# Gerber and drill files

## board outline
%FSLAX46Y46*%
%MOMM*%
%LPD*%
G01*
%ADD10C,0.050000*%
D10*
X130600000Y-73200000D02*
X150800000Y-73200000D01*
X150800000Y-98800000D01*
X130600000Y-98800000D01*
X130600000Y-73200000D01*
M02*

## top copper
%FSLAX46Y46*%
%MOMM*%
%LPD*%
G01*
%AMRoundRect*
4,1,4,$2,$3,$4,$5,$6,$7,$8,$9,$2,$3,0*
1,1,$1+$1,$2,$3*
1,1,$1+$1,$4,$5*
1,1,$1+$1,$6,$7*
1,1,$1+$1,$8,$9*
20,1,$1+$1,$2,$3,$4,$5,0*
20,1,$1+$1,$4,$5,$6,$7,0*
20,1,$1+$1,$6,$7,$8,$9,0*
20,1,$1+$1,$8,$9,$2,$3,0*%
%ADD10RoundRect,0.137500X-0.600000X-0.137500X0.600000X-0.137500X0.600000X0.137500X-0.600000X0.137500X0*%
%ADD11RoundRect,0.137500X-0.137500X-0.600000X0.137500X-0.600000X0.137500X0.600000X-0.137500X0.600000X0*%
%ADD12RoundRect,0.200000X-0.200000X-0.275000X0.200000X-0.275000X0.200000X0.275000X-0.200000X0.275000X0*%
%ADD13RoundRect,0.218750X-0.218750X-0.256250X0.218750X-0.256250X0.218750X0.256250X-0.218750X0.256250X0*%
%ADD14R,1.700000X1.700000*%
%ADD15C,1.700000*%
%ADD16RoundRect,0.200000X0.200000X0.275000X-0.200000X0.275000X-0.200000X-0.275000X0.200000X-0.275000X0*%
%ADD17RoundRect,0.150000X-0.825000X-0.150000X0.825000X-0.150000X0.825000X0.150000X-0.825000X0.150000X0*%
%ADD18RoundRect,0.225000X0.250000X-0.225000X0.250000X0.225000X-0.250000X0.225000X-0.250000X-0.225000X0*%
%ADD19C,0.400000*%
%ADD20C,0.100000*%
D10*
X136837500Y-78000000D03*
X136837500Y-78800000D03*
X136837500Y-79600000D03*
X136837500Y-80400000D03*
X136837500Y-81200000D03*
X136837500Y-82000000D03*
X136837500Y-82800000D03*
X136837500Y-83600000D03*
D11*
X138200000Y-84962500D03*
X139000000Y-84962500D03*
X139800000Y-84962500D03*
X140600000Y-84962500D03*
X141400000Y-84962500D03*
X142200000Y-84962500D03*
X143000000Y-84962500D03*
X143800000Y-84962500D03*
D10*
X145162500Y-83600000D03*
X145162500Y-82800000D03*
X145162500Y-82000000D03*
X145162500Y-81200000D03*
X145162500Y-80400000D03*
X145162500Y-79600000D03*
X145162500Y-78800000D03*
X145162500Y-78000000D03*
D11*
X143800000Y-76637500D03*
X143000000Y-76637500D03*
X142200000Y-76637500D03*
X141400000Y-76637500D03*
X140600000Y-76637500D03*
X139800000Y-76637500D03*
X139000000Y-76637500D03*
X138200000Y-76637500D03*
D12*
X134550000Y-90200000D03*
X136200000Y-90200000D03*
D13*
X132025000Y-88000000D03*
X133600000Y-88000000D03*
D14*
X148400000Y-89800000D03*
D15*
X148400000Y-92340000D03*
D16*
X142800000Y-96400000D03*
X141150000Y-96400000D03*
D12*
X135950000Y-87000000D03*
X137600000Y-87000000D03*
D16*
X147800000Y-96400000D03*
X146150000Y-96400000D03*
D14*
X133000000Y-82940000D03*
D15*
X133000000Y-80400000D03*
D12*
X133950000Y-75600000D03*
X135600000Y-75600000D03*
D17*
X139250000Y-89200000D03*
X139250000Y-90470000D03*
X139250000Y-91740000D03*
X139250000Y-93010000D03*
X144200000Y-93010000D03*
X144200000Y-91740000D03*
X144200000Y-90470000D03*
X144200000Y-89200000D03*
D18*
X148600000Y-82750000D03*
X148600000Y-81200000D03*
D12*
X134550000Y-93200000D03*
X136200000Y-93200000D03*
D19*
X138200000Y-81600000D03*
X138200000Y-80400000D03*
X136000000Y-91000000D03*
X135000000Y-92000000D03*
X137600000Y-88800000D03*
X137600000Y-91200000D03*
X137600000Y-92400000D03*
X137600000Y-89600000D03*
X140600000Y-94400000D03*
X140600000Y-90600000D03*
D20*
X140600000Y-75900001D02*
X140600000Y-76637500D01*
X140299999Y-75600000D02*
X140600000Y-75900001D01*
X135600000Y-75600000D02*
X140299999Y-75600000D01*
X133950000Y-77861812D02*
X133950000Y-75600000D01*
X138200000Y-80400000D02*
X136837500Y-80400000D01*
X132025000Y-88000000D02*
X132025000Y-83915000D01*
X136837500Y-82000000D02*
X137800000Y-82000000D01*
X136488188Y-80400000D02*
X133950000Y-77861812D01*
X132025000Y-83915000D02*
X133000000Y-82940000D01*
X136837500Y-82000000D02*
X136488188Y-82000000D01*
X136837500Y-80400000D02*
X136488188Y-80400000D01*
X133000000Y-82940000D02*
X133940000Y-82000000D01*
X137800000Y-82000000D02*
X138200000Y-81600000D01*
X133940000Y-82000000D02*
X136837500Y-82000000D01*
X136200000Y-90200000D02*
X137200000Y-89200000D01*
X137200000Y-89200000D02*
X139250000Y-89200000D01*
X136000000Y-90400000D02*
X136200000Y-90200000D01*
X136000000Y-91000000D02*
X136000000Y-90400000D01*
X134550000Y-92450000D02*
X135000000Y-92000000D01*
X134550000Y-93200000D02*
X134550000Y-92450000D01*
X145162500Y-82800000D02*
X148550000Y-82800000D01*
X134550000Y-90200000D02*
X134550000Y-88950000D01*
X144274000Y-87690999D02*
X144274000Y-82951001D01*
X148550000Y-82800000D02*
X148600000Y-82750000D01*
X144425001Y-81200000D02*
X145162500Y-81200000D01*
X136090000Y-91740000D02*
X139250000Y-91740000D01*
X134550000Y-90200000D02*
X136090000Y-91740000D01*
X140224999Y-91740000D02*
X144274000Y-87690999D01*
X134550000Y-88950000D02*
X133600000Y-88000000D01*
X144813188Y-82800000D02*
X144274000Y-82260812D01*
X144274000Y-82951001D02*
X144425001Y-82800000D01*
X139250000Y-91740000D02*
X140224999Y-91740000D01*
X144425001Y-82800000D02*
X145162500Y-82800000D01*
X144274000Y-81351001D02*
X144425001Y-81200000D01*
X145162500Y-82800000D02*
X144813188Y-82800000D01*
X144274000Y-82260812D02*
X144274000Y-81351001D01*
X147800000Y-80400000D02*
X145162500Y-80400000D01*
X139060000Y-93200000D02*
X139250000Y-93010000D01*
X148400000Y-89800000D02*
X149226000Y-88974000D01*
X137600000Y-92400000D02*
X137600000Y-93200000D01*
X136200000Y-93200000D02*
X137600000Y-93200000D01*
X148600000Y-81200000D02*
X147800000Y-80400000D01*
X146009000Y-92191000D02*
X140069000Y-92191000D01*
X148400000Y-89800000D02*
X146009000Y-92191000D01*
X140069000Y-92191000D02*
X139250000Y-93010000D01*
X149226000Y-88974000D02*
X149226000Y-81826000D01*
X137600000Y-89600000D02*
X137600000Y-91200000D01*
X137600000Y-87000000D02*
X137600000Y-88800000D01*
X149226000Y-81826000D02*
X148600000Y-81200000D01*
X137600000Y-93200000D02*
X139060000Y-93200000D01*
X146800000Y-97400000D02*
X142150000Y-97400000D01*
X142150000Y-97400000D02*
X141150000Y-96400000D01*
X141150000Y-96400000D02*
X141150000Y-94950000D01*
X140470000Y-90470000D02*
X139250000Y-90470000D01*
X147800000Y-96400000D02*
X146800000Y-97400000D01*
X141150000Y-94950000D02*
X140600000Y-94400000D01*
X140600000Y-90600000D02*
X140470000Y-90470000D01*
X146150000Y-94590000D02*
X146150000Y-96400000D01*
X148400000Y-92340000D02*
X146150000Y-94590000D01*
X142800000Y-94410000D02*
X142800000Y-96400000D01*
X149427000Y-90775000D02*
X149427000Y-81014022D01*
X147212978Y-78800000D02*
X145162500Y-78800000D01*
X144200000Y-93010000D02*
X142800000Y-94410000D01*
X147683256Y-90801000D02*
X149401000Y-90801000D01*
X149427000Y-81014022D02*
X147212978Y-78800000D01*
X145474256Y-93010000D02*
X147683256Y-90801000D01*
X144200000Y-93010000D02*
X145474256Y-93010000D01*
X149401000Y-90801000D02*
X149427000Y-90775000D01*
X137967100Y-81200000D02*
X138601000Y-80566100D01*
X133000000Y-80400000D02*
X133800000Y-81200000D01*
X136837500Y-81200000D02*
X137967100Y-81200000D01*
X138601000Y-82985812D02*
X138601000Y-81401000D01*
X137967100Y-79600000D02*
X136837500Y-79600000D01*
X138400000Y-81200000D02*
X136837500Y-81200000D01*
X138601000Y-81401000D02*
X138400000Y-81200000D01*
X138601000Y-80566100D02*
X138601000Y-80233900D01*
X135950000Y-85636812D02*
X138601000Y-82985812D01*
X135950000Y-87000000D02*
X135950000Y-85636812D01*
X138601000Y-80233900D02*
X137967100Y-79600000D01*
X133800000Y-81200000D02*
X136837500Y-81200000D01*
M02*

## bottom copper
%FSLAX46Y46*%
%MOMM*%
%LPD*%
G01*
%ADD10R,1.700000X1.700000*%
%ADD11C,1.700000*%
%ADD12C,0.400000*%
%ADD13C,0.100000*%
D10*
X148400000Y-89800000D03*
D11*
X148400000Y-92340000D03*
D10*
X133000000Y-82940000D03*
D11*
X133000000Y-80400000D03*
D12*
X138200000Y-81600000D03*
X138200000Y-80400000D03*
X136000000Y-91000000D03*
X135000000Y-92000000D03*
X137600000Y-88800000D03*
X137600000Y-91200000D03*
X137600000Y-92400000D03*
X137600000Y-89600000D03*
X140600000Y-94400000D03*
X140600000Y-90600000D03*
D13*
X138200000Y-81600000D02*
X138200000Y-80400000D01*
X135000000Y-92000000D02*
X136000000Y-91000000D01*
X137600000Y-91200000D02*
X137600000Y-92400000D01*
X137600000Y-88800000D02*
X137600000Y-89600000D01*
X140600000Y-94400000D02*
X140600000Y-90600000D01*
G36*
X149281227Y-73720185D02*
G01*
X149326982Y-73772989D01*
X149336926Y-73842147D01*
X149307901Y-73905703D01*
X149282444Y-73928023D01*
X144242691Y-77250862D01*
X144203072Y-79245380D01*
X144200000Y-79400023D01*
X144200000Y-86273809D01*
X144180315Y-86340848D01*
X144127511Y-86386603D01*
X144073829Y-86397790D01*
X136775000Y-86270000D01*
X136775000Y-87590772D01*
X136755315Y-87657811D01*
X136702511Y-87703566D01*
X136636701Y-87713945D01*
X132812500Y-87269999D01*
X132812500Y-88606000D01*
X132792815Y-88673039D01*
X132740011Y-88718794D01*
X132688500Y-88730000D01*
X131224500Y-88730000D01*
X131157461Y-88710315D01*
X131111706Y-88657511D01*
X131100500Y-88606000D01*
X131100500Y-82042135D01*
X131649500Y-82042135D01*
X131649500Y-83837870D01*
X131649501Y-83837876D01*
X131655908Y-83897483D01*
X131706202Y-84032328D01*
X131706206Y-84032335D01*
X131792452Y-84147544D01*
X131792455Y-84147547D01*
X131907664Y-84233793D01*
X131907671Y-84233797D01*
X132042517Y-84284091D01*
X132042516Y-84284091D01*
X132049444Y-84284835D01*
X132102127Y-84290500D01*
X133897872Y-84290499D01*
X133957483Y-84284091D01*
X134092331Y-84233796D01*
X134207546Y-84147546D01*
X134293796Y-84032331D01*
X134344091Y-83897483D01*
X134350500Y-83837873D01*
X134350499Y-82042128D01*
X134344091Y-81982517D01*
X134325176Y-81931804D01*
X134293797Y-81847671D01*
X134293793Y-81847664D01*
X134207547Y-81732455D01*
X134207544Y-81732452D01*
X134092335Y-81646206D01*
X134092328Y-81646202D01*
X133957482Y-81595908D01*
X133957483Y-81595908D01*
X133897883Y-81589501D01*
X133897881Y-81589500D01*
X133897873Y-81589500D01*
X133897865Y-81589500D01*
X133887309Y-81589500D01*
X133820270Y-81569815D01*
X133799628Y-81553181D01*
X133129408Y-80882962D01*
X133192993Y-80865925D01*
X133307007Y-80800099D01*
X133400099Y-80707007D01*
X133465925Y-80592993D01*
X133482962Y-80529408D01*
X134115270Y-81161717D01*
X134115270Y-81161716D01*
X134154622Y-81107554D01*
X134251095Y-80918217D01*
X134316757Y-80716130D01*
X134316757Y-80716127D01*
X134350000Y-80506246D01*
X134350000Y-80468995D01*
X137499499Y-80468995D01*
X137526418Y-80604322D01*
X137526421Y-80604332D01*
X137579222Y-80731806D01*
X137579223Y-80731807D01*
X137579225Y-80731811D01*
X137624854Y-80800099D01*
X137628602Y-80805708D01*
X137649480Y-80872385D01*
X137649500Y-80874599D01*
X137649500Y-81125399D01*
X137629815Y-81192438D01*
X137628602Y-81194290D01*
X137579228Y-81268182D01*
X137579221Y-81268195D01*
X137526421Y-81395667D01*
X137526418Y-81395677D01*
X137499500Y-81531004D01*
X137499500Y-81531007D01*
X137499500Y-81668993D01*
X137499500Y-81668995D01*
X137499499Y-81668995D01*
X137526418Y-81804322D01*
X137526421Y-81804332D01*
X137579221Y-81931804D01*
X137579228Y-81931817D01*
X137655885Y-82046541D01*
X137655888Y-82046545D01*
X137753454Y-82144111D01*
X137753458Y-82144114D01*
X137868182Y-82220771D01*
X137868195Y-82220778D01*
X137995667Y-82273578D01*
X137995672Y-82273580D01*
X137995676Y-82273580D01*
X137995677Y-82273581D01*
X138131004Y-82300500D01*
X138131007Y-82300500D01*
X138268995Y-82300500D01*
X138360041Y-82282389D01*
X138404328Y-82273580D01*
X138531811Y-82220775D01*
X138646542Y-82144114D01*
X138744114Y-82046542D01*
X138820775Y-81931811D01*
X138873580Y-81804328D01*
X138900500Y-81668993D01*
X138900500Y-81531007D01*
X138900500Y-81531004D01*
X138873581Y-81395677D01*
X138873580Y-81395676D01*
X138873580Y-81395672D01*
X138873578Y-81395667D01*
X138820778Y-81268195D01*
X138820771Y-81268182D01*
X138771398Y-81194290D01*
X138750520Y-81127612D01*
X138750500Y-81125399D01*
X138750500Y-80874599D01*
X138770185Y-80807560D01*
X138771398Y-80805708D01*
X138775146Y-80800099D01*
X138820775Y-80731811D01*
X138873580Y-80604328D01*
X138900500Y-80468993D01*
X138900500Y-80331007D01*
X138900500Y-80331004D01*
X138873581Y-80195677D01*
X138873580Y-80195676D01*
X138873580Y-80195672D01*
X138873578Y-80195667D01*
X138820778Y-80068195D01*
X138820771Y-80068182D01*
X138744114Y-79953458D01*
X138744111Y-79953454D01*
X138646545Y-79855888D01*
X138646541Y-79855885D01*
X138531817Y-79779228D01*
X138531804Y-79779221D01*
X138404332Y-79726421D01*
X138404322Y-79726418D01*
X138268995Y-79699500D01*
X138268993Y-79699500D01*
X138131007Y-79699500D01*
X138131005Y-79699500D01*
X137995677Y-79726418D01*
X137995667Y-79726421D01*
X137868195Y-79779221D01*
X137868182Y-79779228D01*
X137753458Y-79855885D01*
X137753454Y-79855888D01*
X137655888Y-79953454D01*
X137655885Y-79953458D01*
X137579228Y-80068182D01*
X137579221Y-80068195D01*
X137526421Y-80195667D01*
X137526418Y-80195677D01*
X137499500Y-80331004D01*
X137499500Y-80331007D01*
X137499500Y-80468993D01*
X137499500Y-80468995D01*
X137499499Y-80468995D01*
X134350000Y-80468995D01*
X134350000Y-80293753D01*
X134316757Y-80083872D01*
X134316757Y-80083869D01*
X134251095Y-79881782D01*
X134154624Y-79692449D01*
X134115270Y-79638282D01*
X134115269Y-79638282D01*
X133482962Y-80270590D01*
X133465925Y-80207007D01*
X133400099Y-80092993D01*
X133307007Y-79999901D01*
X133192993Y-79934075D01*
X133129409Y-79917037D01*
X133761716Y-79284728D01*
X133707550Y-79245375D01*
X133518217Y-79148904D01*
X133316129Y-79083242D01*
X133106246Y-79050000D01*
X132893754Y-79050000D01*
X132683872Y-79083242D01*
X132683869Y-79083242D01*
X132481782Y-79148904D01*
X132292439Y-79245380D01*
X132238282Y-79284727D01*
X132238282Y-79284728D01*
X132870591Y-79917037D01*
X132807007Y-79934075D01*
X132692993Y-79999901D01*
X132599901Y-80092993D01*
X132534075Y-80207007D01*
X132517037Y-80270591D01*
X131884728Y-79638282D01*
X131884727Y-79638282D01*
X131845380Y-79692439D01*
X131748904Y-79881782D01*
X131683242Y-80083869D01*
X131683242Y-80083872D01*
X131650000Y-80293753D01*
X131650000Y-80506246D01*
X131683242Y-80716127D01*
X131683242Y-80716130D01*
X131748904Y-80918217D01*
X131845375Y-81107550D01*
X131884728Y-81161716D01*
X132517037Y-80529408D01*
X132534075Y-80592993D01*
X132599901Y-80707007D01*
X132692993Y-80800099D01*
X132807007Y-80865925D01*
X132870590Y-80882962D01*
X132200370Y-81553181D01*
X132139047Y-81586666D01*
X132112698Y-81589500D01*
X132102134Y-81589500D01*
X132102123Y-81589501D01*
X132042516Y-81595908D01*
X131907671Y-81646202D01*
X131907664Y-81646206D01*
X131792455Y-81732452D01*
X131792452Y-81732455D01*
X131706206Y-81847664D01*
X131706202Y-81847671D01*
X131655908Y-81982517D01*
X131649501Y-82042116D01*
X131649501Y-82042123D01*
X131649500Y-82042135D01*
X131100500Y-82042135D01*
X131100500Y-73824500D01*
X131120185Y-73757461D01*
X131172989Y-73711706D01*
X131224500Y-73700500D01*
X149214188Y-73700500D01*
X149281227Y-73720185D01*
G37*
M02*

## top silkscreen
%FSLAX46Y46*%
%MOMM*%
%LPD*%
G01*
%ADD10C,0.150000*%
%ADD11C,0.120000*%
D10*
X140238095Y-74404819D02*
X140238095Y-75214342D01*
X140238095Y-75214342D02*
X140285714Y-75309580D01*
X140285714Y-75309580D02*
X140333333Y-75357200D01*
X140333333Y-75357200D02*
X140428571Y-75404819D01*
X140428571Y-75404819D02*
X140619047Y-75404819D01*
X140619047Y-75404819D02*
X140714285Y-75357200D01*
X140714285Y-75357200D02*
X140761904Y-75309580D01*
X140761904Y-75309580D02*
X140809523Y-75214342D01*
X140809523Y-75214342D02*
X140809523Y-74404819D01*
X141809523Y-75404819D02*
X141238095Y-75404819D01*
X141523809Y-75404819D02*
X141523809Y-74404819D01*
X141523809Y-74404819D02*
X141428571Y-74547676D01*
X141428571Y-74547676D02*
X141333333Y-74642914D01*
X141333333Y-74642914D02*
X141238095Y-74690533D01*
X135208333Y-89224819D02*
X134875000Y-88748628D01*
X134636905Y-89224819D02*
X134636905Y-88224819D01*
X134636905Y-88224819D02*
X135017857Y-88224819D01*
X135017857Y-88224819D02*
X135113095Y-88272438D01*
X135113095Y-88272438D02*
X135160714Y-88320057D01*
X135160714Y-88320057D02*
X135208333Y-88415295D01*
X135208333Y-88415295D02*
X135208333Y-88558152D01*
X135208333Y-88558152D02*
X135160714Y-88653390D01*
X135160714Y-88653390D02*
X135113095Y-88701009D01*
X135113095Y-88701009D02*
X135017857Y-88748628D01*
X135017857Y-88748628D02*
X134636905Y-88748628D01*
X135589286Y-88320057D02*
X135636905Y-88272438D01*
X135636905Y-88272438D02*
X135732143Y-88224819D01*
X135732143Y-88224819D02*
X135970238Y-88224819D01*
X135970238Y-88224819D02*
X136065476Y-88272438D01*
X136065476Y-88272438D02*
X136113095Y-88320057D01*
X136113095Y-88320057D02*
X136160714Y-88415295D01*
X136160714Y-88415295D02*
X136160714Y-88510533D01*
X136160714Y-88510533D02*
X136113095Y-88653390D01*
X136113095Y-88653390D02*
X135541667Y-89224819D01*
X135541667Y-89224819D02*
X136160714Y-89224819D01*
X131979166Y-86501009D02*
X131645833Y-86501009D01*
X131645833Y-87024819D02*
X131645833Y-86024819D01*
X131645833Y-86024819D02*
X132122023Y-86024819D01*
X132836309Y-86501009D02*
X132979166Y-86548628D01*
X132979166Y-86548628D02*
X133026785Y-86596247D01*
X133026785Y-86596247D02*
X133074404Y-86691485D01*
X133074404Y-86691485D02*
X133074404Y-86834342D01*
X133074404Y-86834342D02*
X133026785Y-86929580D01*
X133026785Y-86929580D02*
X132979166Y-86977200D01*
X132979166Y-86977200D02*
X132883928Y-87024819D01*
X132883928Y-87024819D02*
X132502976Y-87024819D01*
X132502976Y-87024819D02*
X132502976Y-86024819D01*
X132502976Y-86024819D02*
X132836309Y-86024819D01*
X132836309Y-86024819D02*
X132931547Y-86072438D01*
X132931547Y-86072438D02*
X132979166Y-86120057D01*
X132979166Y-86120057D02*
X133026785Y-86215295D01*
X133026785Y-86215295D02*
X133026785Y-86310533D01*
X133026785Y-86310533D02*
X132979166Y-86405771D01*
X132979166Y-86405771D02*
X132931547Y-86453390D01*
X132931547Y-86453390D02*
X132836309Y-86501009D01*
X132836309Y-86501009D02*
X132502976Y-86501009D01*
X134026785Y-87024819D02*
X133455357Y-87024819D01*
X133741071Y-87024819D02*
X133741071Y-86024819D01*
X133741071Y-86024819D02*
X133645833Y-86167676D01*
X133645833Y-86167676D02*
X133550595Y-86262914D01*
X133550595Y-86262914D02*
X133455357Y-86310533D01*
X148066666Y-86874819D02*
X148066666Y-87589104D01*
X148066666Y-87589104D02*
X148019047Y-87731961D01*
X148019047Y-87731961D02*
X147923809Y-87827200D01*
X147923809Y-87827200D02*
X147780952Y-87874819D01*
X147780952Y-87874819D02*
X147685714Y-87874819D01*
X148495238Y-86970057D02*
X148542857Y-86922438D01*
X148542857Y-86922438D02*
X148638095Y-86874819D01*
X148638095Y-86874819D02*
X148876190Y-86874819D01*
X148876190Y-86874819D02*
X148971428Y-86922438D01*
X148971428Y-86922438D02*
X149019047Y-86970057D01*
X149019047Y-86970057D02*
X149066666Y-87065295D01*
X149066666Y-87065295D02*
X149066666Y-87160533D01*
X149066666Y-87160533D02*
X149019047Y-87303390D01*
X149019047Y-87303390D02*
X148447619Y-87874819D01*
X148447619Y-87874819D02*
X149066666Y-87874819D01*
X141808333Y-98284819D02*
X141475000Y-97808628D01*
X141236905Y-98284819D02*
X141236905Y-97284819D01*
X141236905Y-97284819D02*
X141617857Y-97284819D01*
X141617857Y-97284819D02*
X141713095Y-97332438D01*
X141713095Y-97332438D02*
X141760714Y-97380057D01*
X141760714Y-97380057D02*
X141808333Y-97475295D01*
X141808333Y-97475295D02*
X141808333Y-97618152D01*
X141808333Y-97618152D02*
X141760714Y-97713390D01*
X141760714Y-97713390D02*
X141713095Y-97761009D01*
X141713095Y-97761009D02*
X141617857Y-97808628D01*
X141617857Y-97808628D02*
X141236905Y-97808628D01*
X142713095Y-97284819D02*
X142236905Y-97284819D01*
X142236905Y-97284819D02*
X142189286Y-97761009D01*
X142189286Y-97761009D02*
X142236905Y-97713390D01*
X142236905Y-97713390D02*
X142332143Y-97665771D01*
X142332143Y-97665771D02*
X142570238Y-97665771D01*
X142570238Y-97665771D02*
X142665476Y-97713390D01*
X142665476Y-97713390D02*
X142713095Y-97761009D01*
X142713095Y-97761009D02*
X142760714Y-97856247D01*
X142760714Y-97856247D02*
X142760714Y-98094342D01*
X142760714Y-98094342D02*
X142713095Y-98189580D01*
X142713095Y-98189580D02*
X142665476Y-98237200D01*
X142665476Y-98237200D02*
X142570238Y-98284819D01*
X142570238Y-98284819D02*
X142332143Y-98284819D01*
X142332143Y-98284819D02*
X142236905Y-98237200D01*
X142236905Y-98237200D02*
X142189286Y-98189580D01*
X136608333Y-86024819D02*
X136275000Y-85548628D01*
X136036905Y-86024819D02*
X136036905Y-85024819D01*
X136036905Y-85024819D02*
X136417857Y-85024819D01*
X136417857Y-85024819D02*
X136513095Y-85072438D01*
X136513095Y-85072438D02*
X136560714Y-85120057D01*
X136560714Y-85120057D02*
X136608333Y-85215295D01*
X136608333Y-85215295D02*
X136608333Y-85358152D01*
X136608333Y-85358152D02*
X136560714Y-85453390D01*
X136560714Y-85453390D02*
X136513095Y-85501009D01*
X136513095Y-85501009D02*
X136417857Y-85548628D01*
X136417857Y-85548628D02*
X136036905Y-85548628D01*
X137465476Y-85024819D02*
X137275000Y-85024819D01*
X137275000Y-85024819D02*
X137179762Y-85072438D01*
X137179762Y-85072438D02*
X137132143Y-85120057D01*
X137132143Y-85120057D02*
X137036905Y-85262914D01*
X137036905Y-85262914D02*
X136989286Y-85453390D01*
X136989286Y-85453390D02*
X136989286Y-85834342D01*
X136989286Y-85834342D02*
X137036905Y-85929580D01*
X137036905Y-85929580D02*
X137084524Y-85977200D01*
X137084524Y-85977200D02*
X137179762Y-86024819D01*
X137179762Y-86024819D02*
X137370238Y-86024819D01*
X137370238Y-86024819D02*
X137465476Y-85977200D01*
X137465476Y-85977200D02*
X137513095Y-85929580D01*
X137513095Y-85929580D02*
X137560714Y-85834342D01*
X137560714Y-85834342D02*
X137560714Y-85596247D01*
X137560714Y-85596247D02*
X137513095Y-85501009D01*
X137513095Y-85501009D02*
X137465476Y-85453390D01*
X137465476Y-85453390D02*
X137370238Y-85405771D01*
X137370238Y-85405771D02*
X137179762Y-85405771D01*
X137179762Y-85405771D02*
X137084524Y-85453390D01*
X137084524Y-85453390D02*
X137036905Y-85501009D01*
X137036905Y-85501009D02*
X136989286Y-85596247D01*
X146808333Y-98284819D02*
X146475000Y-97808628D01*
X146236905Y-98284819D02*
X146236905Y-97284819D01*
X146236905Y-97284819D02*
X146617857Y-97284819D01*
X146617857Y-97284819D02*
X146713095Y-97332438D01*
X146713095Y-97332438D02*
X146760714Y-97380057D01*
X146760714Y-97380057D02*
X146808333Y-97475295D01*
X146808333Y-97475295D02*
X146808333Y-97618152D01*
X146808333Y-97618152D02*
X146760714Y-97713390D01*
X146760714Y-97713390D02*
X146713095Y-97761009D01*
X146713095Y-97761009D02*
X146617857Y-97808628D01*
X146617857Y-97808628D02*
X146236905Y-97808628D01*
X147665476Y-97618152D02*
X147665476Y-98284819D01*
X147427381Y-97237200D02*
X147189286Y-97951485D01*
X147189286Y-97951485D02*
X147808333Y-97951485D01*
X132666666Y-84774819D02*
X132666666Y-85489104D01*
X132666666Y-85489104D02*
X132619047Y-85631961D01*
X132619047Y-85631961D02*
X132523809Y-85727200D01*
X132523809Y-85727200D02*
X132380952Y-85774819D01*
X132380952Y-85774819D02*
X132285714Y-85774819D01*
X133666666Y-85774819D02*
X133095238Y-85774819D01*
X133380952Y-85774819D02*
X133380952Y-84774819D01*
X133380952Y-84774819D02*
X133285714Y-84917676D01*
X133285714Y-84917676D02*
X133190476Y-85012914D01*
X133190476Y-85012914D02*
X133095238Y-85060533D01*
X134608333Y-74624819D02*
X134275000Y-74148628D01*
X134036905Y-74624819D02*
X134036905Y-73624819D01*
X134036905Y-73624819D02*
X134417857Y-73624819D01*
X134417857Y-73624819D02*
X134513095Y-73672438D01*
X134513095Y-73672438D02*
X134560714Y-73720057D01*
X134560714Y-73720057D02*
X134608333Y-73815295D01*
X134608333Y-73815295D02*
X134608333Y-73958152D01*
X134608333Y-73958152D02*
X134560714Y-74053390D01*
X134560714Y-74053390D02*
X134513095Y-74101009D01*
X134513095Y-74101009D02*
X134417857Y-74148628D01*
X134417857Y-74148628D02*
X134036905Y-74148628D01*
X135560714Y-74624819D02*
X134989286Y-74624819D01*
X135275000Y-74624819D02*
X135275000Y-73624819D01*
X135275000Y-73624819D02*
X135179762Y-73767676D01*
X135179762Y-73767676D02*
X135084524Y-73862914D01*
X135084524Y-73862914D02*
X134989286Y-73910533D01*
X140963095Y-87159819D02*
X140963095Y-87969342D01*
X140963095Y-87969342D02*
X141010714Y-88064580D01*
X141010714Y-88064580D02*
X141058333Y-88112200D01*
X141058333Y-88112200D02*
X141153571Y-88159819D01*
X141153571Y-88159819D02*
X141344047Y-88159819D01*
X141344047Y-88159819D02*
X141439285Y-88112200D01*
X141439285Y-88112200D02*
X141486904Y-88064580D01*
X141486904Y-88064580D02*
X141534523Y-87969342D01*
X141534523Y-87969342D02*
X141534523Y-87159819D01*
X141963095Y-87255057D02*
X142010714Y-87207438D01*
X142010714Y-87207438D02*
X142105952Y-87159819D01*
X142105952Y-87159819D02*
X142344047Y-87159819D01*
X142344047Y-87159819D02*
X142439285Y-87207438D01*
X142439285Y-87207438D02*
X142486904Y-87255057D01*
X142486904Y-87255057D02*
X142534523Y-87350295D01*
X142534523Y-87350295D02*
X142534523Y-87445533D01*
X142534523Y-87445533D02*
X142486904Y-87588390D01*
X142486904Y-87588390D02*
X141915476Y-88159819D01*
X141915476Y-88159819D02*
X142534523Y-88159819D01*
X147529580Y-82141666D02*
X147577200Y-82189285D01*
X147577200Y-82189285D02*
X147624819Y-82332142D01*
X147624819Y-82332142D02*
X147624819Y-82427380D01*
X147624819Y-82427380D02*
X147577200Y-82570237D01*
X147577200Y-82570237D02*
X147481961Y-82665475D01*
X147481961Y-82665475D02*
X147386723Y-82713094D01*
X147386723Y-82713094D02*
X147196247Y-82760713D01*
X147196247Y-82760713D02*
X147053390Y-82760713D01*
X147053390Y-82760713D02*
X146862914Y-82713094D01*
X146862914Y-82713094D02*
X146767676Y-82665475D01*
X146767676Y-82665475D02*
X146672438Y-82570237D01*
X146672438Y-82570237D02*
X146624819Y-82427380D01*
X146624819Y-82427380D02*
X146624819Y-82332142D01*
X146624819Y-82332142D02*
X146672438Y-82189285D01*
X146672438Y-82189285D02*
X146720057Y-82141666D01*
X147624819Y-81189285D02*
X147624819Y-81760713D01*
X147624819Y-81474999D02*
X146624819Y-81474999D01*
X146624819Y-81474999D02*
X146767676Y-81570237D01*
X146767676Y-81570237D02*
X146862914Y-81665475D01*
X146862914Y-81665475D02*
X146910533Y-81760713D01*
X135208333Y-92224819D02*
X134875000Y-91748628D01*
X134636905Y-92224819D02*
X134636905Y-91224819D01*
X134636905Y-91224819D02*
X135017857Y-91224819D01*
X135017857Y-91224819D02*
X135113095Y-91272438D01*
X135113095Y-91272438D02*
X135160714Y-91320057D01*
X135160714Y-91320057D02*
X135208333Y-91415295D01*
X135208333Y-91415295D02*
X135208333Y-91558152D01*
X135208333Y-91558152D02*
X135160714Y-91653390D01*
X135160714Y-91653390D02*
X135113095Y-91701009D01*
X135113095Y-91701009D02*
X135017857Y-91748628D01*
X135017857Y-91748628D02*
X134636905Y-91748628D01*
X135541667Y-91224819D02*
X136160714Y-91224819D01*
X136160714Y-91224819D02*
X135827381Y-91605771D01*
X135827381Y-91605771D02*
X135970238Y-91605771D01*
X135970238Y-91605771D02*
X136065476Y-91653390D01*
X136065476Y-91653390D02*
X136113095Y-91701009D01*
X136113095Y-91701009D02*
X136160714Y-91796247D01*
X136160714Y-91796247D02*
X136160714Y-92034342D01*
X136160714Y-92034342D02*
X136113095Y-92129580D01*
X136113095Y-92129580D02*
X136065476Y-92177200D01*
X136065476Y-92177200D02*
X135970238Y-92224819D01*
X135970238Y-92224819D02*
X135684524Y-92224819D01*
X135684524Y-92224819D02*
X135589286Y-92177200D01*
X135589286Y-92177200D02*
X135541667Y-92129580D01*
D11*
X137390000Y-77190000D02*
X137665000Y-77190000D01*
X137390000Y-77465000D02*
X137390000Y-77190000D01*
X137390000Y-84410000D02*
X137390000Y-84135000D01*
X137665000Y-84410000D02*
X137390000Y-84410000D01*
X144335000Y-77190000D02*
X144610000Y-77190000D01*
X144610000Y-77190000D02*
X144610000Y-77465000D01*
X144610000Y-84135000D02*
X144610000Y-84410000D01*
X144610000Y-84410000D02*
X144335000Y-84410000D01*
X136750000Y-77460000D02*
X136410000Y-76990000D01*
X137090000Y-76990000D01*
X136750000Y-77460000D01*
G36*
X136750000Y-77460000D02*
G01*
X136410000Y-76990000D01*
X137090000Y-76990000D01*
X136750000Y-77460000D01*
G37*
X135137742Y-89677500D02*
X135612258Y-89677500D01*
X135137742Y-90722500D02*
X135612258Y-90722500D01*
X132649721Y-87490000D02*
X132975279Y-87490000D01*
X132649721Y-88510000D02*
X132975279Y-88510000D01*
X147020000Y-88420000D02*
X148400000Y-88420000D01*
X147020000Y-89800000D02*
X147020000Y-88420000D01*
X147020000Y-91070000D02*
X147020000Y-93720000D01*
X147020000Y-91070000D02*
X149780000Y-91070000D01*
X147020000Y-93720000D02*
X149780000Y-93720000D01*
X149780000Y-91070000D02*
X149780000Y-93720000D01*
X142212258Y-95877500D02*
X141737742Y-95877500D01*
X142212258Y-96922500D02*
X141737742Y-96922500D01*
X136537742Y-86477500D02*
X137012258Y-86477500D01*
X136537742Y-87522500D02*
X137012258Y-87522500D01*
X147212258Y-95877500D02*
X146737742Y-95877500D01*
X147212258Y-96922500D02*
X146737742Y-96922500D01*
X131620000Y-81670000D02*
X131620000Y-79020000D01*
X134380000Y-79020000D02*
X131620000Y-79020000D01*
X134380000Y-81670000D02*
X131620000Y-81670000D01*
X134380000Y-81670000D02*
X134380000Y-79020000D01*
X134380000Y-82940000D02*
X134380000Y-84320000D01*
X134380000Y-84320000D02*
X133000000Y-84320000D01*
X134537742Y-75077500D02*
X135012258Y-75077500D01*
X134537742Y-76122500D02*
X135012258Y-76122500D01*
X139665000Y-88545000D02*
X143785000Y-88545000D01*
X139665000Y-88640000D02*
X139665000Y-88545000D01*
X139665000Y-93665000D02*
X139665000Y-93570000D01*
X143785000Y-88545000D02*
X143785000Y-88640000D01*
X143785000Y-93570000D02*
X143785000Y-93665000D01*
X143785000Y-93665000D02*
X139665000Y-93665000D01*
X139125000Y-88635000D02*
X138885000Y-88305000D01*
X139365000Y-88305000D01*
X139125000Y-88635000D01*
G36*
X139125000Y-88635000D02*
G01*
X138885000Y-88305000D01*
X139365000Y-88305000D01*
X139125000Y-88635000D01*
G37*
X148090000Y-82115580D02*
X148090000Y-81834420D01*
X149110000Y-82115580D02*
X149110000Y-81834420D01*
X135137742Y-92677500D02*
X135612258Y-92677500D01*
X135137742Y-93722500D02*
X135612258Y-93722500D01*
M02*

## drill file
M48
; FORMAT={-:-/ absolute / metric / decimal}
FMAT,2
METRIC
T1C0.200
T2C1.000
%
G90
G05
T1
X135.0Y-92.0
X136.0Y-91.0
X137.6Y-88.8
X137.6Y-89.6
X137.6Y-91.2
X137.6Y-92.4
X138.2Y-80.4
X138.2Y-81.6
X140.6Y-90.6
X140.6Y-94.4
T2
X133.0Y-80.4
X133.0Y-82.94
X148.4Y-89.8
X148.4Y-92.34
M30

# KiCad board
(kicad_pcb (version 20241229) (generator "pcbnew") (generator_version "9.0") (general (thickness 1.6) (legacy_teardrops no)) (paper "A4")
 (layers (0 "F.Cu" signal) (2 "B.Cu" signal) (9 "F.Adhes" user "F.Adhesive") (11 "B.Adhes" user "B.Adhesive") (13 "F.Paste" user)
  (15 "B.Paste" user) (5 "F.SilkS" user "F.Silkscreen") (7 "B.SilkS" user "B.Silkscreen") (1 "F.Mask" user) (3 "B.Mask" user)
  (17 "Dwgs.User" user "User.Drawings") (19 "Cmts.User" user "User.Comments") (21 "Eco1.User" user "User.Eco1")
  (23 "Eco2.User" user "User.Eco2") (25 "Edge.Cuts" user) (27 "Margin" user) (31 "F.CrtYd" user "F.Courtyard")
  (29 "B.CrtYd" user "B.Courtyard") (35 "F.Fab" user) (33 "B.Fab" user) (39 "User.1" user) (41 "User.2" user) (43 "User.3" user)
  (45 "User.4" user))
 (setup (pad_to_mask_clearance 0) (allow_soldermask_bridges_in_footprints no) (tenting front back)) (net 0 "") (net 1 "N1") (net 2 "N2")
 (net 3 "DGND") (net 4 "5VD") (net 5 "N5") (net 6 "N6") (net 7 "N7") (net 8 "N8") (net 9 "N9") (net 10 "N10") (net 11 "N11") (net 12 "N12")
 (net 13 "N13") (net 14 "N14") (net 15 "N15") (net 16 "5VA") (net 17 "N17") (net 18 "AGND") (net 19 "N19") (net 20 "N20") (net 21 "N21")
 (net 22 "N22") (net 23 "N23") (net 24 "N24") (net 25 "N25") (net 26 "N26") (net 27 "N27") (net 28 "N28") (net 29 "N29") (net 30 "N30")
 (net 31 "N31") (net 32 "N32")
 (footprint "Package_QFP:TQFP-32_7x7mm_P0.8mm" (layer "F.Cu") (at 141 80.8)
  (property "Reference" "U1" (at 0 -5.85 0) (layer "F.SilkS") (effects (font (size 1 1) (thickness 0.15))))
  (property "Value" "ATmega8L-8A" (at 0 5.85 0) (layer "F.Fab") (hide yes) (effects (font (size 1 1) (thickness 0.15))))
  (fp_line (start -3.61 -3.61) (end -3.335 -3.61) (stroke (width 0.12) (type solid)) (layer "F.SilkS"))
  (fp_line (start -3.61 -3.335) (end -3.61 -3.61) (stroke (width 0.12) (type solid)) (layer "F.SilkS"))
  (fp_line (start -3.61 3.61) (end -3.61 3.335) (stroke (width 0.12) (type solid)) (layer "F.SilkS"))
  (fp_line (start -3.335 3.61) (end -3.61 3.61) (stroke (width 0.12) (type solid)) (layer "F.SilkS"))
  (fp_line (start 3.335 -3.61) (end 3.61 -3.61) (stroke (width 0.12) (type solid)) (layer "F.SilkS"))
  (fp_line (start 3.61 -3.61) (end 3.61 -3.335) (stroke (width 0.12) (type solid)) (layer "F.SilkS"))
  (fp_line (start 3.61 3.335) (end 3.61 3.61) (stroke (width 0.12) (type solid)) (layer "F.SilkS"))
  (fp_line (start 3.61 3.61) (end 3.335 3.61) (stroke (width 0.12) (type solid)) (layer "F.SilkS"))
  (fp_poly (pts (xy -4.25 -3.34) (xy -4.59 -3.81) (xy -3.91 -3.81)) (stroke (width 0.12) (type solid)) (fill yes) (layer "F.SilkS"))
  (pad "1" smd roundrect (at -4.1625 -2.8) (size 1.475 0.55) (layers "F.Cu" "F.Mask" "F.Paste") (roundrect_rratio 0.25) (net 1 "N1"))
  (pad "2" smd roundrect (at -4.1625 -2) (size 1.475 0.55) (layers "F.Cu" "F.Mask" "F.Paste") (roundrect_rratio 0.25) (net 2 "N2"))
  (pad "3" smd roundrect (at -4.1625 -1.2) (size 1.475 0.55) (layers "F.Cu" "F.Mask" "F.Paste") (roundrect_rratio 0.25) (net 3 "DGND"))
  (pad "4" smd roundrect (at -4.1625 -0.4) (size 1.475 0.55) (layers "F.Cu" "F.Mask" "F.Paste") (roundrect_rratio 0.25) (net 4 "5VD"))
  (pad "5" smd roundrect (at -4.1625 0.4) (size 1.475 0.55) (layers "F.Cu" "F.Mask" "F.Paste") (roundrect_rratio 0.25) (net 3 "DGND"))
  (pad "6" smd roundrect (at -4.1625 1.2) (size 1.475 0.55) (layers "F.Cu" "F.Mask" "F.Paste") (roundrect_rratio 0.25) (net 4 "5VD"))
  (pad "7" smd roundrect (at -4.1625 2) (size 1.475 0.55) (layers "F.Cu" "F.Mask" "F.Paste") (roundrect_rratio 0.25) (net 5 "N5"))
  (pad "8" smd roundrect (at -4.1625 2.8) (size 1.475 0.55) (layers "F.Cu" "F.Mask" "F.Paste") (roundrect_rratio 0.25) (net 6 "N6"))
  (pad "9" smd roundrect (at -2.8 4.1625) (size 0.55 1.475) (layers "F.Cu" "F.Mask" "F.Paste") (roundrect_rratio 0.25) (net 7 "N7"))
  (pad "10" smd roundrect (at -2 4.1625) (size 0.55 1.475) (layers "F.Cu" "F.Mask" "F.Paste") (roundrect_rratio 0.25) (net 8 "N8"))
  (pad "11" smd roundrect (at -1.2 4.1625) (size 0.55 1.475) (layers "F.Cu" "F.Mask" "F.Paste") (roundrect_rratio 0.25) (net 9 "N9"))
  (pad "12" smd roundrect (at -0.4 4.1625) (size 0.55 1.475) (layers "F.Cu" "F.Mask" "F.Paste") (roundrect_rratio 0.25) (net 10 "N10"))
  (pad "13" smd roundrect (at 0.4 4.1625) (size 0.55 1.475) (layers "F.Cu" "F.Mask" "F.Paste") (roundrect_rratio 0.25) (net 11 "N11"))
  (pad "14" smd roundrect (at 1.2 4.1625) (size 0.55 1.475) (layers "F.Cu" "F.Mask" "F.Paste") (roundrect_rratio 0.25) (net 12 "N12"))
  (pad "15" smd roundrect (at 2 4.1625) (size 0.55 1.475) (layers "F.Cu" "F.Mask" "F.Paste") (roundrect_rratio 0.25) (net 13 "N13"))
  (pad "16" smd roundrect (at 2.8 4.1625) (size 0.55 1.475) (layers "F.Cu" "F.Mask" "F.Paste") (roundrect_rratio 0.25) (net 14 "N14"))
  (pad "17" smd roundrect (at 4.1625 2.8) (size 1.475 0.55) (layers "F.Cu" "F.Mask" "F.Paste") (roundrect_rratio 0.25) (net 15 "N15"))
  (pad "18" smd roundrect (at 4.1625 2) (size 1.475 0.55) (layers "F.Cu" "F.Mask" "F.Paste") (roundrect_rratio 0.25) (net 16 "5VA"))
  (pad "19" smd roundrect (at 4.1625 1.2) (size 1.475 0.55) (layers "F.Cu" "F.Mask" "F.Paste") (roundrect_rratio 0.25) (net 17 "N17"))
  (pad "20" smd roundrect (at 4.1625 0.4) (size 1.475 0.55) (layers "F.Cu" "F.Mask" "F.Paste") (roundrect_rratio 0.25) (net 16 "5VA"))
  (pad "21" smd roundrect (at 4.1625 -0.4) (size 1.475 0.55) (layers "F.Cu" "F.Mask" "F.Paste") (roundrect_rratio 0.25) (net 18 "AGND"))
  (pad "22" smd roundrect (at 4.1625 -1.2) (size 1.475 0.55) (layers "F.Cu" "F.Mask" "F.Paste") (roundrect_rratio 0.25) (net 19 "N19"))
  (pad "23" smd roundrect (at 4.1625 -2) (size 1.475 0.55) (layers "F.Cu" "F.Mask" "F.Paste") (roundrect_rratio 0.25) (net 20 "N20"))
  (pad "24" smd roundrect (at 4.1625 -2.8) (size 1.475 0.55) (layers "F.Cu" "F.Mask" "F.Paste") (roundrect_rratio 0.25) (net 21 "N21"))
  (pad "25" smd roundrect (at 2.8 -4.1625) (size 0.55 1.475) (layers "F.Cu" "F.Mask" "F.Paste") (roundrect_rratio 0.25) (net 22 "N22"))
  (pad "26" smd roundrect (at 2 -4.1625) (size 0.55 1.475) (layers "F.Cu" "F.Mask" "F.Paste") (roundrect_rratio 0.25) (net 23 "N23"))
  (pad "27" smd roundrect (at 1.2 -4.1625) (size 0.55 1.475) (layers "F.Cu" "F.Mask" "F.Paste") (roundrect_rratio 0.25) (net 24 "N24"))
  (pad "28" smd roundrect (at 0.4 -4.1625) (size 0.55 1.475) (layers "F.Cu" "F.Mask" "F.Paste") (roundrect_rratio 0.25) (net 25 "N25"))
  (pad "29" smd roundrect (at -0.4 -4.1625) (size 0.55 1.475) (layers "F.Cu" "F.Mask" "F.Paste") (roundrect_rratio 0.25) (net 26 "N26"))
  (pad "30" smd roundrect (at -1.2 -4.1625) (size 0.55 1.475) (layers "F.Cu" "F.Mask" "F.Paste") (roundrect_rratio 0.25) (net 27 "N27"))
  (pad "31" smd roundrect (at -2 -4.1625) (size 0.55 1.475) (layers "F.Cu" "F.Mask" "F.Paste") (roundrect_rratio 0.25) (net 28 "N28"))
  (pad "32" smd roundrect (at -2.8 -4.1625) (size 0.55 1.475) (layers "F.Cu" "F.Mask" "F.Paste") (roundrect_rratio 0.25) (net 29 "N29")))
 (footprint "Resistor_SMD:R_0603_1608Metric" (layer "F.Cu") (at 135.375 90.2)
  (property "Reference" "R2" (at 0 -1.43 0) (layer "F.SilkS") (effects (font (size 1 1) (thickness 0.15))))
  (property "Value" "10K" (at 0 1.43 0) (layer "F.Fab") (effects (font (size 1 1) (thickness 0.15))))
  (fp_line (start -0.237258 -0.5225) (end 0.237258 -0.5225) (stroke (width 0.12) (type solid)) (layer "F.SilkS"))
  (fp_line (start -0.237258 0.5225) (end 0.237258 0.5225) (stroke (width 0.12) (type solid)) (layer "F.SilkS"))
  (pad "1" smd roundrect (at -0.825 0) (size 0.8 0.95) (layers "F.Cu" "F.Mask" "F.Paste") (roundrect_rratio 0.25) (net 16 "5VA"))
  (pad "2" smd roundrect (at 0.825 0) (size 0.8 0.95) (layers "F.Cu" "F.Mask" "F.Paste") (roundrect_rratio 0.25) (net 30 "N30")))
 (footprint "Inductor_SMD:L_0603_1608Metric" (layer "F.Cu") (at 132.8125 88)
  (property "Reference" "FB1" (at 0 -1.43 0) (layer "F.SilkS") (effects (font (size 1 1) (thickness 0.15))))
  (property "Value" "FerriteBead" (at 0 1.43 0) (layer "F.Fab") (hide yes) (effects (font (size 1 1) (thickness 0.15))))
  (fp_line (start -0.162779 -0.51) (end 0.162779 -0.51) (stroke (width 0.12) (type solid)) (layer "F.SilkS"))
  (fp_line (start -0.162779 0.51) (end 0.162779 0.51) (stroke (width 0.12) (type solid)) (layer "F.SilkS"))
  (pad "1" smd roundrect (at -0.7875 0) (size 0.875 0.95) (layers "F.Cu" "F.Mask" "F.Paste") (roundrect_rratio 0.25) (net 4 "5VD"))
  (pad "2" smd roundrect (at 0.7875 0) (size 0.875 0.95) (layers "F.Cu" "F.Mask" "F.Paste") (roundrect_rratio 0.25) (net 16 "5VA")))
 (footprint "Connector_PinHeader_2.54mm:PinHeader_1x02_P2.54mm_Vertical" (layer "F.Cu") (at 148.4 89.8)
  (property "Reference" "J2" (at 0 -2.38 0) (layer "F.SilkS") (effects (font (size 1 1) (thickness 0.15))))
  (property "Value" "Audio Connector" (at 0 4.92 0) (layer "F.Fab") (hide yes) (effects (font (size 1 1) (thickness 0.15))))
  (fp_line (start -1.38 -1.38) (end 0 -1.38) (stroke (width 0.12) (type solid)) (layer "F.SilkS"))
  (fp_line (start -1.38 0) (end -1.38 -1.38) (stroke (width 0.12) (type solid)) (layer "F.SilkS"))
  (fp_line (start -1.38 1.27) (end -1.38 3.92) (stroke (width 0.12) (type solid)) (layer "F.SilkS"))
  (fp_line (start -1.38 1.27) (end 1.38 1.27) (stroke (width 0.12) (type solid)) (layer "F.SilkS"))
  (fp_line (start -1.38 3.92) (end 1.38 3.92) (stroke (width 0.12) (type solid)) (layer "F.SilkS"))
  (fp_line (start 1.38 1.27) (end 1.38 3.92) (stroke (width 0.12) (type solid)) (layer "F.SilkS"))
  (pad "1" thru_hole rect (at 0 0) (size 1.7 1.7) (drill 1) (layers "*.Cu" "*.Mask") (remove_unused_layers no) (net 18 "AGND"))
  (pad "2" thru_hole circle (at 0 2.54) (size 1.7 1.7) (drill 1) (layers "*.Cu" "*.Mask") (remove_unused_layers no) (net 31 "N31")))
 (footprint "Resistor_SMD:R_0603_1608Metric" (layer "F.Cu") (at 141.975 96.4 180)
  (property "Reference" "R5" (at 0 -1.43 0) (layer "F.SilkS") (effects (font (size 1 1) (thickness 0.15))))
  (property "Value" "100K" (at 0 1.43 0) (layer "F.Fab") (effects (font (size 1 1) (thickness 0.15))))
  (fp_line (start -0.237258 0.5225) (end 0.237258 0.5225) (stroke (width 0.12) (type solid)) (layer "F.SilkS"))
  (fp_line (start -0.237258 -0.5225) (end 0.237258 -0.5225) (stroke (width 0.12) (type solid)) (layer "F.SilkS"))
  (pad "1" smd roundrect (at -0.825 0 180) (size 0.8 0.95) (layers "F.Cu" "F.Mask" "F.Paste") (roundrect_rratio 0.25) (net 20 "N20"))
  (pad "2" smd roundrect (at 0.825 0 180) (size 0.8 0.95) (layers "F.Cu" "F.Mask" "F.Paste") (roundrect_rratio 0.25) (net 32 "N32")))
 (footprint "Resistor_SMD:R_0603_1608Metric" (layer "F.Cu") (at 136.775 87)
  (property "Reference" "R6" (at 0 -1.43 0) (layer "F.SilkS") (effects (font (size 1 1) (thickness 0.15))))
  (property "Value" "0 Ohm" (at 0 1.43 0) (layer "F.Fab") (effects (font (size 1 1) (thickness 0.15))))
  (fp_line (start -0.237258 -0.5225) (end 0.237258 -0.5225) (stroke (width 0.12) (type solid)) (layer "F.SilkS"))
  (fp_line (start -0.237258 0.5225) (end 0.237258 0.5225) (stroke (width 0.12) (type solid)) (layer "F.SilkS"))
  (pad "1" smd roundrect (at -0.825 0) (size 0.8 0.95) (layers "F.Cu" "F.Mask" "F.Paste") (roundrect_rratio 0.25) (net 3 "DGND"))
  (pad "2" smd roundrect (at 0.825 0) (size 0.8 0.95) (layers "F.Cu" "F.Mask" "F.Paste") (roundrect_rratio 0.25) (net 18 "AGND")))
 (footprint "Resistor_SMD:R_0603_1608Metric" (layer "F.Cu") (at 146.975 96.4 180)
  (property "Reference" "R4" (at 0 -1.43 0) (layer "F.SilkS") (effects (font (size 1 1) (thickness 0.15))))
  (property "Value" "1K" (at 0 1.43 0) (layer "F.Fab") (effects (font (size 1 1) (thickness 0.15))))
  (fp_line (start -0.237258 0.5225) (end 0.237258 0.5225) (stroke (width 0.12) (type solid)) (layer "F.SilkS"))
  (fp_line (start -0.237258 -0.5225) (end 0.237258 -0.5225) (stroke (width 0.12) (type solid)) (layer "F.SilkS"))
  (pad "1" smd roundrect (at -0.825 0 180) (size 0.8 0.95) (layers "F.Cu" "F.Mask" "F.Paste") (roundrect_rratio 0.25) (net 32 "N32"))
  (pad "2" smd roundrect (at 0.825 0 180) (size 0.8 0.95) (layers "F.Cu" "F.Mask" "F.Paste") (roundrect_rratio 0.25) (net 31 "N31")))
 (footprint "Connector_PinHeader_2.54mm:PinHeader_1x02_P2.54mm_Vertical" (layer "F.Cu") (at 133 82.94 180)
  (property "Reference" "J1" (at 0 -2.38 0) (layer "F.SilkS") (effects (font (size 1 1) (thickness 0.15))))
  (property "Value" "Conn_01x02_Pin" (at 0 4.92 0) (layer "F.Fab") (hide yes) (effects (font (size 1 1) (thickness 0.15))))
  (fp_line (start 1.38 1.27) (end 1.38 3.92) (stroke (width 0.12) (type solid)) (layer "F.SilkS"))
  (fp_line (start -1.38 3.92) (end 1.38 3.92) (stroke (width 0.12) (type solid)) (layer "F.SilkS"))
  (fp_line (start -1.38 1.27) (end 1.38 1.27) (stroke (width 0.12) (type solid)) (layer "F.SilkS"))
  (fp_line (start -1.38 1.27) (end -1.38 3.92) (stroke (width 0.12) (type solid)) (layer "F.SilkS"))
  (fp_line (start -1.38 0) (end -1.38 -1.38) (stroke (width 0.12) (type solid)) (layer "F.SilkS"))
  (fp_line (start -1.38 -1.38) (end 0 -1.38) (stroke (width 0.12) (type solid)) (layer "F.SilkS"))
  (pad "1" thru_hole rect (at 0 0 180) (size 1.7 1.7) (drill 1) (layers "*.Cu" "*.Mask") (remove_unused_layers no) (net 4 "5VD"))
  (pad "2" thru_hole circle (at 0 2.54 180) (size 1.7 1.7) (drill 1) (layers "*.Cu" "*.Mask") (remove_unused_layers no) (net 3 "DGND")))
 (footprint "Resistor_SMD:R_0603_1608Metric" (layer "F.Cu") (at 134.775 75.6)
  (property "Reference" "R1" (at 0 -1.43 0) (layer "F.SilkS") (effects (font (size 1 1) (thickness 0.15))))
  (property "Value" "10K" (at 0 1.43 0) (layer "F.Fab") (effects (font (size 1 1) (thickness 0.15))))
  (fp_line (start -0.237258 -0.5225) (end 0.237258 -0.5225) (stroke (width 0.12) (type solid)) (layer "F.SilkS"))
  (fp_line (start -0.237258 0.5225) (end 0.237258 0.5225) (stroke (width 0.12) (type solid)) (layer "F.SilkS"))
  (pad "1" smd roundrect (at -0.825 0) (size 0.8 0.95) (layers "F.Cu" "F.Mask" "F.Paste") (roundrect_rratio 0.25) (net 4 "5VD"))
  (pad "2" smd roundrect (at 0.825 0) (size 0.8 0.95) (layers "F.Cu" "F.Mask" "F.Paste") (roundrect_rratio 0.25) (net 26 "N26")))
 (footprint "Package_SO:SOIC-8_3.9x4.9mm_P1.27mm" (layer "F.Cu") (at 141.725 91.105)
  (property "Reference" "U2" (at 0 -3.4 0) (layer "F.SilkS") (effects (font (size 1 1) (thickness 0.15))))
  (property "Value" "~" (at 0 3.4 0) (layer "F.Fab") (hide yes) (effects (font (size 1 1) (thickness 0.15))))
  (fp_line (start -2.06 -2.56) (end 2.06 -2.56) (stroke (width 0.12) (type solid)) (layer "F.SilkS"))
  (fp_line (start -2.06 -2.465) (end -2.06 -2.56) (stroke (width 0.12) (type solid)) (layer "F.SilkS"))
  (fp_line (start -2.06 2.56) (end -2.06 2.465) (stroke (width 0.12) (type solid)) (layer "F.SilkS"))
  (fp_line (start 2.06 -2.56) (end 2.06 -2.465) (stroke (width 0.12) (type solid)) (layer "F.SilkS"))
  (fp_line (start 2.06 2.465) (end 2.06 2.56) (stroke (width 0.12) (type solid)) (layer "F.SilkS"))
  (fp_line (start 2.06 2.56) (end -2.06 2.56) (stroke (width 0.12) (type solid)) (layer "F.SilkS"))
  (fp_poly (pts (xy -2.6 -2.47) (xy -2.84 -2.8) (xy -2.36 -2.8)) (stroke (width 0.12) (type solid)) (fill yes) (layer "F.SilkS"))
  (pad "1" smd roundrect (at -2.475 -1.905) (size 1.95 0.6) (layers "F.Cu" "F.Mask" "F.Paste") (roundrect_rratio 0.25) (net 30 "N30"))
  (pad "2" smd roundrect (at -2.475 -0.635) (size 1.95 0.6) (layers "F.Cu" "F.Mask" "F.Paste") (roundrect_rratio 0.25) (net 32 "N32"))
  (pad "3" smd roundrect (at -2.475 0.635) (size 1.95 0.6) (layers "F.Cu" "F.Mask" "F.Paste") (roundrect_rratio 0.25) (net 16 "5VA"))
  (pad "4" smd roundrect (at -2.475 1.905) (size 1.95 0.6) (layers "F.Cu" "F.Mask" "F.Paste") (roundrect_rratio 0.25) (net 18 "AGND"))
  (pad "5" smd roundrect (at 2.475 1.905) (size 1.95 0.6) (layers "F.Cu" "F.Mask" "F.Paste") (roundrect_rratio 0.25) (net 20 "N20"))
  (pad "6" smd roundrect (at 2.475 0.635) (size 1.95 0.6) (layers "F.Cu" "F.Mask" "F.Paste") (roundrect_rratio 0.25))
  (pad "7" smd roundrect (at 2.475 -0.635) (size 1.95 0.6) (layers "F.Cu" "F.Mask" "F.Paste") (roundrect_rratio 0.25))
  (pad "8" smd roundrect (at 2.475 -1.905) (size 1.95 0.6) (layers "F.Cu" "F.Mask" "F.Paste") (roundrect_rratio 0.25)))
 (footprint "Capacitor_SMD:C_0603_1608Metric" (layer "F.Cu") (at 148.6 81.975 90)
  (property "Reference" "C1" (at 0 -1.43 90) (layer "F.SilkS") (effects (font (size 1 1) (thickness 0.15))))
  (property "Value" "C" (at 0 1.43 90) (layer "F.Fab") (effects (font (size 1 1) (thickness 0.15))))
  (fp_line (start -0.14058 -0.51) (end 0.14058 -0.51) (stroke (width 0.12) (type solid)) (layer "F.SilkS"))
  (fp_line (start -0.14058 0.51) (end 0.14058 0.51) (stroke (width 0.12) (type solid)) (layer "F.SilkS"))
  (pad "1" smd roundrect (at -0.775 0 90) (size 0.9 0.95) (layers "F.Cu" "F.Mask" "F.Paste") (roundrect_rratio 0.25) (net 16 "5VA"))
  (pad "2" smd roundrect (at 0.775 0 90) (size 0.9 0.95) (layers "F.Cu" "F.Mask" "F.Paste") (roundrect_rratio 0.25) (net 18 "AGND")))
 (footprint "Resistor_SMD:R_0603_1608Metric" (layer "F.Cu") (at 135.375 93.2)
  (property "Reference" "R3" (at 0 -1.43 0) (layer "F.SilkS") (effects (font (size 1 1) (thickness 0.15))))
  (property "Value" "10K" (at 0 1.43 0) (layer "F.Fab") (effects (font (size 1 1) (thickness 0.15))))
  (fp_line (start -0.237258 -0.5225) (end 0.237258 -0.5225) (stroke (width 0.12) (type solid)) (layer "F.SilkS"))
  (fp_line (start -0.237258 0.5225) (end 0.237258 0.5225) (stroke (width 0.12) (type solid)) (layer "F.SilkS"))
  (pad "1" smd roundrect (at -0.825 0) (size 0.8 0.95) (layers "F.Cu" "F.Mask" "F.Paste") (roundrect_rratio 0.25) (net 30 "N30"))
  (pad "2" smd roundrect (at 0.825 0) (size 0.8 0.95) (layers "F.Cu" "F.Mask" "F.Paste") (roundrect_rratio 0.25) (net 18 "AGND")))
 (gr_rect (start 130.6 73.2) (end 150.8 98.8) (stroke (width 0.05) (type default)) (fill no) (layer "Edge.Cuts"))
 (segment (start 140.6 75.900001) (end 140.6 76.6375) (width 0.1) (layer "F.Cu") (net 26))
 (segment (start 140.299999 75.6) (end 140.6 75.900001) (width 0.1) (layer "F.Cu") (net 26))
 (segment (start 135.6 75.6) (end 140.299999 75.6) (width 0.1) (layer "F.Cu") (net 26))
 (segment (start 133.95 77.861812) (end 133.95 75.6) (width 0.1) (layer "F.Cu") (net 4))
 (segment (start 138.2 80.4) (end 136.8375 80.4) (width 0.1) (layer "F.Cu") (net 4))
 (segment (start 132.025 88) (end 132.025 83.915) (width 0.1) (layer "F.Cu") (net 4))
 (segment (start 136.8375 82) (end 137.8 82) (width 0.1) (layer "F.Cu") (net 4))
 (segment (start 136.488188 80.4) (end 133.95 77.861812) (width 0.1) (layer "F.Cu") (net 4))
 (segment (start 132.025 83.915) (end 133 82.94) (width 0.1) (layer "F.Cu") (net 4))
 (segment (start 136.8375 82) (end 136.488188 82) (width 0.1) (layer "F.Cu") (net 4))
 (segment (start 136.8375 80.4) (end 136.488188 80.4) (width 0.1) (layer "F.Cu") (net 4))
 (segment (start 133 82.94) (end 133.94 82) (width 0.1) (layer "F.Cu") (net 4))
 (segment (start 137.8 82) (end 138.2 81.6) (width 0.1) (layer "F.Cu") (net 4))
 (segment (start 133.94 82) (end 136.8375 82) (width 0.1) (layer "F.Cu") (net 4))
 (via (at 138.2 81.6) (size 0.4) (drill 0.2) (layers "F.Cu" "B.Cu") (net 4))
 (via (at 138.2 80.4) (size 0.4) (drill 0.2) (layers "F.Cu" "B.Cu") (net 4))
 (segment (start 138.2 81.6) (end 138.2 80.4) (width 0.1) (layer "B.Cu") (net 4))
 (segment (start 136.2 90.2) (end 137.2 89.2) (width 0.1) (layer "F.Cu") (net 30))
 (segment (start 137.2 89.2) (end 139.25 89.2) (width 0.1) (layer "F.Cu") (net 30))
 (segment (start 136 90.4) (end 136.2 90.2) (width 0.1) (layer "F.Cu") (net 30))
 (segment (start 136 91) (end 136 90.4) (width 0.1) (layer "F.Cu") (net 30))
 (segment (start 134.55 92.45) (end 135 92) (width 0.1) (layer "F.Cu") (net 30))
 (segment (start 134.55 93.2) (end 134.55 92.45) (width 0.1) (layer "F.Cu") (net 30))
 (via (at 136 91) (size 0.4) (drill 0.2) (layers "F.Cu" "B.Cu") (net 30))
 (via (at 135 92) (size 0.4) (drill 0.2) (layers "F.Cu" "B.Cu") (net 30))
 (segment (start 135 92) (end 136 91) (width 0.1) (layer "B.Cu") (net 30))
 (segment (start 145.1625 82.8) (end 148.55 82.8) (width 0.1) (layer "F.Cu") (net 16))
 (segment (start 134.55 90.2) (end 134.55 88.95) (width 0.1) (layer "F.Cu") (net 16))
 (segment (start 144.274 87.690999) (end 144.274 82.951001) (width 0.1) (layer "F.Cu") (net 16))
 (segment (start 148.55 82.8) (end 148.6 82.75) (width 0.1) (layer "F.Cu") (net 16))
 (segment (start 144.425001 81.2) (end 145.1625 81.2) (width 0.1) (layer "F.Cu") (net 16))
 (segment (start 136.09 91.74) (end 139.25 91.74) (width 0.1) (layer "F.Cu") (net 16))
 (segment (start 134.55 90.2) (end 136.09 91.74) (width 0.1) (layer "F.Cu") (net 16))
 (segment (start 140.224999 91.74) (end 144.274 87.690999) (width 0.1) (layer "F.Cu") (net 16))
 (segment (start 134.55 88.95) (end 133.6 88) (width 0.1) (layer "F.Cu") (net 16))
 (segment (start 144.813188 82.8) (end 144.274 82.260812) (width 0.1) (layer "F.Cu") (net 16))
 (segment (start 144.274 82.951001) (end 144.425001 82.8) (width 0.1) (layer "F.Cu") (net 16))
 (segment (start 139.25 91.74) (end 140.224999 91.74) (width 0.1) (layer "F.Cu") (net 16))
 (segment (start 144.425001 82.8) (end 145.1625 82.8) (width 0.1) (layer "F.Cu") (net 16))
 (segment (start 144.274 81.351001) (end 144.425001 81.2) (width 0.1) (layer "F.Cu") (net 16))
 (segment (start 145.1625 82.8) (end 144.813188 82.8) (width 0.1) (layer "F.Cu") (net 16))
 (segment (start 144.274 82.260812) (end 144.274 81.351001) (width 0.1) (layer "F.Cu") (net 16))
 (segment (start 147.8 80.4) (end 145.1625 80.4) (width 0.1) (layer "F.Cu") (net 18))
 (segment (start 139.06 93.2) (end 139.25 93.01) (width 0.1) (layer "F.Cu") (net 18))
 (segment (start 148.4 89.8) (end 149.226 88.974) (width 0.1) (layer "F.Cu") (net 18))
 (segment (start 137.6 92.4) (end 137.6 93.2) (width 0.1) (layer "F.Cu") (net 18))
 (segment (start 136.2 93.2) (end 137.6 93.2) (width 0.1) (layer "F.Cu") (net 18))
 (segment (start 148.6 81.2) (end 147.8 80.4) (width 0.1) (layer "F.Cu") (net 18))
 (segment (start 146.009 92.191) (end 140.069 92.191) (width 0.1) (layer "F.Cu") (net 18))
 (segment (start 148.4 89.8) (end 146.009 92.191) (width 0.1) (layer "F.Cu") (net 18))
 (segment (start 140.069 92.191) (end 139.25 93.01) (width 0.1) (layer "F.Cu") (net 18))
 (segment (start 149.226 88.974) (end 149.226 81.826) (width 0.1) (layer "F.Cu") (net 18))
 (segment (start 137.6 89.6) (end 137.6 91.2) (width 0.1) (layer "F.Cu") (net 18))
 (segment (start 137.6 87) (end 137.6 88.8) (width 0.1) (layer "F.Cu") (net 18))
 (segment (start 149.226 81.826) (end 148.6 81.2) (width 0.1) (layer "F.Cu") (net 18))
 (segment (start 137.6 93.2) (end 139.06 93.2) (width 0.1) (layer "F.Cu") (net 18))
 (via (at 137.6 88.8) (size 0.4) (drill 0.2) (layers "F.Cu" "B.Cu") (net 18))
 (via (at 137.6 91.2) (size 0.4) (drill 0.2) (layers "F.Cu" "B.Cu") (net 18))
 (via (at 137.6 92.4) (size 0.4) (drill 0.2) (layers "F.Cu" "B.Cu") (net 18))
 (via (at 137.6 89.6) (size 0.4) (drill 0.2) (layers "F.Cu" "B.Cu") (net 18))
 (segment (start 137.6 91.2) (end 137.6 92.4) (width 0.1) (layer "B.Cu") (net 18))
 (segment (start 137.6 88.8) (end 137.6 89.6) (width 0.1) (layer "B.Cu") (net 18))
 (segment (start 146.8 97.4) (end 142.15 97.4) (width 0.1) (layer "F.Cu") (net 32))
 (segment (start 142.15 97.4) (end 141.15 96.4) (width 0.1) (layer "F.Cu") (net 32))
 (segment (start 141.15 96.4) (end 141.15 94.95) (width 0.1) (layer "F.Cu") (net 32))
 (segment (start 140.47 90.47) (end 139.25 90.47) (width 0.1) (layer "F.Cu") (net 32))
 (segment (start 147.8 96.4) (end 146.8 97.4) (width 0.1) (layer "F.Cu") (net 32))
 (segment (start 141.15 94.95) (end 140.6 94.4) (width 0.1) (layer "F.Cu") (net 32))
 (segment (start 140.6 90.6) (end 140.47 90.47) (width 0.1) (layer "F.Cu") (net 32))
 (via (at 140.6 94.4) (size 0.4) (drill 0.2) (layers "F.Cu" "B.Cu") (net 32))
 (via (at 140.6 90.6) (size 0.4) (drill 0.2) (layers "F.Cu" "B.Cu") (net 32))
 (segment (start 140.6 94.4) (end 140.6 90.6) (width 0.1) (layer "B.Cu") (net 32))
 (segment (start 146.15 94.59) (end 146.15 96.4) (width 0.1) (layer "F.Cu") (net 31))
 (segment (start 148.4 92.34) (end 146.15 94.59) (width 0.1) (layer "F.Cu") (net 31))
 (segment (start 142.8 94.41) (end 142.8 96.4) (width 0.1) (layer "F.Cu") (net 20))
 (segment (start 149.427 90.775) (end 149.427 81.014022) (width 0.1) (layer "F.Cu") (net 20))
 (segment (start 147.212978 78.8) (end 145.1625 78.8) (width 0.1) (layer "F.Cu") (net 20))
 (segment (start 144.2 93.01) (end 142.8 94.41) (width 0.1) (layer "F.Cu") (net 20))
 (segment (start 147.683256 90.801) (end 149.401 90.801) (width 0.1) (layer "F.Cu") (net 20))
 (segment (start 149.427 81.014022) (end 147.212978 78.8) (width 0.1) (layer "F.Cu") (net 20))
 (segment (start 145.474256 93.01) (end 147.683256 90.801) (width 0.1) (layer "F.Cu") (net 20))
 (segment (start 144.2 93.01) (end 145.474256 93.01) (width 0.1) (layer "F.Cu") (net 20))
 (segment (start 149.401 90.801) (end 149.427 90.775) (width 0.1) (layer "F.Cu") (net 20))
 (segment (start 137.9671 81.2) (end 138.601 80.5661) (width 0.1) (layer "F.Cu") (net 3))
 (segment (start 133 80.4) (end 133.8 81.2) (width 0.1) (layer "F.Cu") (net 3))
 (segment (start 136.8375 81.2) (end 137.9671 81.2) (width 0.1) (layer "F.Cu") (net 3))
 (segment (start 138.601 82.985812) (end 138.601 81.401) (width 0.1) (layer "F.Cu") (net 3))
 (segment (start 137.9671 79.6) (end 136.8375 79.6) (width 0.1) (layer "F.Cu") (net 3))
 (segment (start 138.4 81.2) (end 136.8375 81.2) (width 0.1) (layer "F.Cu") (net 3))
 (segment (start 138.601 81.401) (end 138.4 81.2) (width 0.1) (layer "F.Cu") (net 3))
 (segment (start 138.601 80.5661) (end 138.601 80.2339) (width 0.1) (layer "F.Cu") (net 3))
 (segment (start 135.95 85.636812) (end 138.601 82.985812) (width 0.1) (layer "F.Cu") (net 3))
 (segment (start 135.95 87) (end 135.95 85.636812) (width 0.1) (layer "F.Cu") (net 3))
 (segment (start 138.601 80.2339) (end 137.9671 79.6) (width 0.1) (layer "F.Cu") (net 3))
 (segment (start 133.8 81.2) (end 136.8375 81.2) (width 0.1) (layer "F.Cu") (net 3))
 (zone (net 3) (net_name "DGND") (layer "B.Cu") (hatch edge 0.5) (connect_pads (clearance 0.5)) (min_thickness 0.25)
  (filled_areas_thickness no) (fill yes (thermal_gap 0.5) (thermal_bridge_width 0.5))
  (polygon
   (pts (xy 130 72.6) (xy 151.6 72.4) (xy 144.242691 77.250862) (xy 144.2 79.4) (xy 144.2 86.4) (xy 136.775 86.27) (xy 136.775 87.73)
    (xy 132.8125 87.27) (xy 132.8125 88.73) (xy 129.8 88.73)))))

